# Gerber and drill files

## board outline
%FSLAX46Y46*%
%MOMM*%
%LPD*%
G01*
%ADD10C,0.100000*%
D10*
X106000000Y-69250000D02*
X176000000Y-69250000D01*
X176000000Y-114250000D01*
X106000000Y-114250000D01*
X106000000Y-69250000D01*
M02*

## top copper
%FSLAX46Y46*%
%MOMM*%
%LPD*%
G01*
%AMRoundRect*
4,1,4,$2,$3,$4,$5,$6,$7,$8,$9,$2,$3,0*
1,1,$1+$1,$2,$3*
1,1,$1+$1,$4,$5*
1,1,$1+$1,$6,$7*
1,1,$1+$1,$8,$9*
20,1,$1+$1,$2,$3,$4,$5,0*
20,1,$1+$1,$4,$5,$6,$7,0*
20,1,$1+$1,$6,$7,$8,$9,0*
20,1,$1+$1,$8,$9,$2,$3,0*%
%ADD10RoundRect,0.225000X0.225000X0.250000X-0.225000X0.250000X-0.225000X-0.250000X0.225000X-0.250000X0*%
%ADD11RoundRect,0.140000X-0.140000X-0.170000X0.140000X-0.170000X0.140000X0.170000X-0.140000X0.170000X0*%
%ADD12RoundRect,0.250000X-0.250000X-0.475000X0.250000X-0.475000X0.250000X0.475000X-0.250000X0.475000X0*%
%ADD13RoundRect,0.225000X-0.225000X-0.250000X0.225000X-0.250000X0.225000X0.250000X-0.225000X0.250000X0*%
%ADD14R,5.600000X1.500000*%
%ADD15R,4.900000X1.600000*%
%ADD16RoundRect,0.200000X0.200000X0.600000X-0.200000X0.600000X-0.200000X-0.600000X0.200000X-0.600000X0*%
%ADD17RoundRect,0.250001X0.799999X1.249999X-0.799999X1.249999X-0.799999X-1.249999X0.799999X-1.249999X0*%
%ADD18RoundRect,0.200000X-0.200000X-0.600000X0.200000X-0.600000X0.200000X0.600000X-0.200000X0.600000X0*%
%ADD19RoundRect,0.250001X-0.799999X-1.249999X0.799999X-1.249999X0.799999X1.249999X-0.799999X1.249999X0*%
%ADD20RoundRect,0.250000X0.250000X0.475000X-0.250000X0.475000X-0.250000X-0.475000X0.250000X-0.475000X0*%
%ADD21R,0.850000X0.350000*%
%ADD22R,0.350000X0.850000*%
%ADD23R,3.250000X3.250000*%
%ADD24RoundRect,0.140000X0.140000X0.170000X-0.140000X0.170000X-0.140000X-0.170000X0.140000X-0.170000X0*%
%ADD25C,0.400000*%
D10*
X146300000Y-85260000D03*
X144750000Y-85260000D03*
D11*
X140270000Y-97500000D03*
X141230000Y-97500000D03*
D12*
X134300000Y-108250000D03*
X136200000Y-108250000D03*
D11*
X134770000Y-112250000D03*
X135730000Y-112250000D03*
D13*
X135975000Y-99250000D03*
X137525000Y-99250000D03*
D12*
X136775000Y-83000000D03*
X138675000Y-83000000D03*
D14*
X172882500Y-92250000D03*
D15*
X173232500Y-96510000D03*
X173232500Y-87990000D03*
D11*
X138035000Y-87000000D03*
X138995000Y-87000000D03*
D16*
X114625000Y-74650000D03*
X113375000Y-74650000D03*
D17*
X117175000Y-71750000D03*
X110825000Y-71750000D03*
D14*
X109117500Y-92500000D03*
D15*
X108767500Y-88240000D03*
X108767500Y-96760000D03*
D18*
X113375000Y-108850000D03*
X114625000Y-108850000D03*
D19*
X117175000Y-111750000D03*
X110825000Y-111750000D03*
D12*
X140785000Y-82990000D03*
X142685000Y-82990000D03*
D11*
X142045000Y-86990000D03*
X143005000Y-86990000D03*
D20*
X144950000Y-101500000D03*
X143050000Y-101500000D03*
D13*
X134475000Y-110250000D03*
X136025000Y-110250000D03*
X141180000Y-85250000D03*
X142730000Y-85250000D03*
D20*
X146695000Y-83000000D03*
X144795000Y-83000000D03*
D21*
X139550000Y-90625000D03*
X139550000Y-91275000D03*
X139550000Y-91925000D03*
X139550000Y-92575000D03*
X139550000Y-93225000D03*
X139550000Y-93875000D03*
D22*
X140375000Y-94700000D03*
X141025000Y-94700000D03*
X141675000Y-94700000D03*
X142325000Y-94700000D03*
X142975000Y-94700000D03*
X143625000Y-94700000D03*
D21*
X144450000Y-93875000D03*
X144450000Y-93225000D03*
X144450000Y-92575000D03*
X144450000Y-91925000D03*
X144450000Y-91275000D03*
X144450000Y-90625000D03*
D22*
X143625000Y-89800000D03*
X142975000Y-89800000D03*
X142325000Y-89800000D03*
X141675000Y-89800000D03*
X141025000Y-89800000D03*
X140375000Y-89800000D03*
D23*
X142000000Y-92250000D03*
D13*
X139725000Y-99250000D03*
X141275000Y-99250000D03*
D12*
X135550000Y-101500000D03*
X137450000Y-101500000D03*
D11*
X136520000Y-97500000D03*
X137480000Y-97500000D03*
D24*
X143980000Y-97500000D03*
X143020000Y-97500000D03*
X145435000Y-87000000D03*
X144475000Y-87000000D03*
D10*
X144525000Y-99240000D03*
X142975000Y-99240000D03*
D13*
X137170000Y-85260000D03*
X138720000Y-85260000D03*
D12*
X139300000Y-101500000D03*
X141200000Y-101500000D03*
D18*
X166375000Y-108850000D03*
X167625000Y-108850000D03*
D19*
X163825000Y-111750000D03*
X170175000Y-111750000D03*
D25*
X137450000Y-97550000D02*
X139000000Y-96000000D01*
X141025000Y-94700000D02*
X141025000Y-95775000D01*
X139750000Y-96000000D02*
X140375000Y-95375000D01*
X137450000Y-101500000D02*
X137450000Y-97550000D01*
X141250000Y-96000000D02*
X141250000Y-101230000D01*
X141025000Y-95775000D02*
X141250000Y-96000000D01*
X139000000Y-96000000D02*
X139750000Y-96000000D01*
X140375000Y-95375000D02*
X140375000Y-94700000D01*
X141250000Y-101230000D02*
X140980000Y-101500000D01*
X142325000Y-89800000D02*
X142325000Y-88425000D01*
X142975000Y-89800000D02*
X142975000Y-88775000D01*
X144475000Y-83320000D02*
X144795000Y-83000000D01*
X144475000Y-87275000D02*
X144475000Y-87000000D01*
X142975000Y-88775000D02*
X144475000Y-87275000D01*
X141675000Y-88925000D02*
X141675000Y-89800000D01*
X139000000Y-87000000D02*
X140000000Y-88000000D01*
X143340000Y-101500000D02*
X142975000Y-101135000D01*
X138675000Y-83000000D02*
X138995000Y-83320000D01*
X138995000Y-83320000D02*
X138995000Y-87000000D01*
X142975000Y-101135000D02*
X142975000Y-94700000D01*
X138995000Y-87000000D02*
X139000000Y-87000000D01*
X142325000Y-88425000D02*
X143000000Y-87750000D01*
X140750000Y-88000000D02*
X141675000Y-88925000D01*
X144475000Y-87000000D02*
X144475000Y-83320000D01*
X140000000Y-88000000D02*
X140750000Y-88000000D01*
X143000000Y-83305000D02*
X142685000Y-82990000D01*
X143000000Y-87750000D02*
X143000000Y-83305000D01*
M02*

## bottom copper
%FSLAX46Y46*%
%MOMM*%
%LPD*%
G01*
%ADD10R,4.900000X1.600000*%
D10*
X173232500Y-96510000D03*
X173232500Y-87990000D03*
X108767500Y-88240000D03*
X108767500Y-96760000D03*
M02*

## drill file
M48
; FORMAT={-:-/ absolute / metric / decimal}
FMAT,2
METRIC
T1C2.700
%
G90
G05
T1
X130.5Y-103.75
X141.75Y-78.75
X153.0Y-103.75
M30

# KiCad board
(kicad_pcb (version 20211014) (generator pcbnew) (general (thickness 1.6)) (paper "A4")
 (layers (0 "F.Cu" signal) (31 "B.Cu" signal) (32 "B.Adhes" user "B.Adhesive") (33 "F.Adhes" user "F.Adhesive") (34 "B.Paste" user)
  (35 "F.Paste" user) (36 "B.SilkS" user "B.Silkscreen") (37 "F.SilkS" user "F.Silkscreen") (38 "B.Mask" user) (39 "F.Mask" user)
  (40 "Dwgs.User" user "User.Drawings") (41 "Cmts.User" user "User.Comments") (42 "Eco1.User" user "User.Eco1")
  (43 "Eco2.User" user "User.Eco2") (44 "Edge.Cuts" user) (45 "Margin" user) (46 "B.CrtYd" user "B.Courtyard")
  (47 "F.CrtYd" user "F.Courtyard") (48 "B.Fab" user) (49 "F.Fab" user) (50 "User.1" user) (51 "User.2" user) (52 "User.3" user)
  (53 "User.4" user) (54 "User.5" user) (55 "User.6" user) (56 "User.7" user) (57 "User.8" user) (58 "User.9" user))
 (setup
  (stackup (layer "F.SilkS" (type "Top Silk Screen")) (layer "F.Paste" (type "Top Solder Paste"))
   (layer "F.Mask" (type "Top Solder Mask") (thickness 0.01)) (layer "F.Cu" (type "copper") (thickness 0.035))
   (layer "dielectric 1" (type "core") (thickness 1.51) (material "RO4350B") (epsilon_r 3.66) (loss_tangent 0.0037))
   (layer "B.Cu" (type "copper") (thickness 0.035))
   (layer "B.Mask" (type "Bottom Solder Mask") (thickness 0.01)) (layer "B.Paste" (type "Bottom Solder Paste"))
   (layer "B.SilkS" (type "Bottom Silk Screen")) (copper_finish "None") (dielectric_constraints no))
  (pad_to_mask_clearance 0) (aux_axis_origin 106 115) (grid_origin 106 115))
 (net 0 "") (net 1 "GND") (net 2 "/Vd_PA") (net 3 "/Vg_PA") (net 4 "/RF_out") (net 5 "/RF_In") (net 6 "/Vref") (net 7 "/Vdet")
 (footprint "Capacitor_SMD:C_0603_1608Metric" (layer "F.Cu") (at 145.525 85.26 180)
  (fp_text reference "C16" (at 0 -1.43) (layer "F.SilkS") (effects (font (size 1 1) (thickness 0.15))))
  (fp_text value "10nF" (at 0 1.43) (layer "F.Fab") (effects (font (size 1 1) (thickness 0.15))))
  (pad "1" smd roundrect (at -0.775 0 180) (size 0.9 0.95) (layers "F.Cu" "F.Paste" "F.Mask") (roundrect_rratio 0.25) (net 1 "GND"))
  (pad "2" smd roundrect (at 0.775 0 180) (size 0.9 0.95) (layers "F.Cu" "F.Paste" "F.Mask") (roundrect_rratio 0.25) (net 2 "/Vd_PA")))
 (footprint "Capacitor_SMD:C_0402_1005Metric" (layer "F.Cu") (at 140.75 97.5)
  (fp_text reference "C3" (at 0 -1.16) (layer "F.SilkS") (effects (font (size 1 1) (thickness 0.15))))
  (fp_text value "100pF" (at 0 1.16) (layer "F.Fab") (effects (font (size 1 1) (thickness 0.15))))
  (pad "1" smd roundrect (at -0.48 0) (size 0.56 0.62) (layers "F.Cu" "F.Paste" "F.Mask") (roundrect_rratio 0.25) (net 1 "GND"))
  (pad "2" smd roundrect (at 0.48 0) (size 0.56 0.62) (layers "F.Cu" "F.Paste" "F.Mask") (roundrect_rratio 0.25) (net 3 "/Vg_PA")))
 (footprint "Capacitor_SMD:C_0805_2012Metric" (layer "F.Cu") (at 135.25 108.25)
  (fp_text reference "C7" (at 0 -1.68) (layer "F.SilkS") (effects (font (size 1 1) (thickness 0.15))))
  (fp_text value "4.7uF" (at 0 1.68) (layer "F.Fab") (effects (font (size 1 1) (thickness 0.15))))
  (pad "1" smd roundrect (at -0.95 0) (size 1 1.45) (layers "F.Cu" "F.Paste" "F.Mask") (roundrect_rratio 0.25) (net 1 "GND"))
  (pad "2" smd roundrect (at 0.95 0) (size 1 1.45) (layers "F.Cu" "F.Paste" "F.Mask") (roundrect_rratio 0.25) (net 3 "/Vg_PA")))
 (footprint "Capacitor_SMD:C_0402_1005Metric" (layer "F.Cu") (at 135.25 112.25)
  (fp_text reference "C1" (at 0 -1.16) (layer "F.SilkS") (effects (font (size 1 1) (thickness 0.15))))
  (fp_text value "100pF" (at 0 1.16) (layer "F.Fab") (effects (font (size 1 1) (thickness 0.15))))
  (pad "1" smd roundrect (at -0.48 0) (size 0.56 0.62) (layers "F.Cu" "F.Paste" "F.Mask") (roundrect_rratio 0.25) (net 1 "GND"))
  (pad "2" smd roundrect (at 0.48 0) (size 0.56 0.62) (layers "F.Cu" "F.Paste" "F.Mask") (roundrect_rratio 0.25) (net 3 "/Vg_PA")))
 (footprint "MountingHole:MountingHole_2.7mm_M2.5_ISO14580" (layer "F.Cu") (at 141.75 78.75)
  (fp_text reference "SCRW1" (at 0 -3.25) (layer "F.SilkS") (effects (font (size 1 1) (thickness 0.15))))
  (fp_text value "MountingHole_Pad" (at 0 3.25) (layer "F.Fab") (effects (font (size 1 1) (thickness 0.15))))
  (pad "" np_thru_hole circle (at 0 0) (size 2.7 2.7) (drill 2.7) (layers *.Cu *.Mask)))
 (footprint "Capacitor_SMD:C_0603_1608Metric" (layer "F.Cu") (at 136.75 99.25)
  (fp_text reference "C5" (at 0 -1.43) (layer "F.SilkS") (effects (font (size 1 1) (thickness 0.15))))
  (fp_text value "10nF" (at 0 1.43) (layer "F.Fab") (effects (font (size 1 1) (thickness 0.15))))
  (pad "1" smd roundrect (at -0.775 0) (size 0.9 0.95) (layers "F.Cu" "F.Paste" "F.Mask") (roundrect_rratio 0.25) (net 1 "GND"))
  (pad "2" smd roundrect (at 0.775 0) (size 0.9 0.95) (layers "F.Cu" "F.Paste" "F.Mask") (roundrect_rratio 0.25) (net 3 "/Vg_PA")))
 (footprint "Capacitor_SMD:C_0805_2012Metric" (layer "F.Cu") (at 137.725 83)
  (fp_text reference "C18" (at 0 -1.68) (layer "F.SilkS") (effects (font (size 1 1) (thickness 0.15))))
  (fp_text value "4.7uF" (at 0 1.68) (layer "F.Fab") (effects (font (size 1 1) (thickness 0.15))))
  (pad "1" smd roundrect (at -0.95 0) (size 1 1.45) (layers "F.Cu" "F.Paste" "F.Mask") (roundrect_rratio 0.25) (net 1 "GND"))
  (pad "2" smd roundrect (at 0.95 0) (size 1 1.45) (layers "F.Cu" "F.Paste" "F.Mask") (roundrect_rratio 0.25) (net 2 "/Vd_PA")))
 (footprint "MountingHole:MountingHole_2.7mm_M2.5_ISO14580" (layer "F.Cu") (at 130.5 103.75)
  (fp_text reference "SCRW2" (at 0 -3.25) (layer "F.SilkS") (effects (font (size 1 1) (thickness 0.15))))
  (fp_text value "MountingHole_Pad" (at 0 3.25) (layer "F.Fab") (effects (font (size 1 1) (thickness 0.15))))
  (pad "" np_thru_hole circle (at 0 0) (size 2.7 2.7) (drill 2.7) (layers *.Cu *.Mask)))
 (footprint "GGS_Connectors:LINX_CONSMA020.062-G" (layer "F.Cu") (at 175.6825 92.25 90)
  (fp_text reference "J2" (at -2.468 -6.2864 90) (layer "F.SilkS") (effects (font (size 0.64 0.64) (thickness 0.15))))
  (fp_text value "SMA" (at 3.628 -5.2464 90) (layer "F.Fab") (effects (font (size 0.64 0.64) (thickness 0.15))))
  (pad "1" smd rect (at 0 -2.8 90) (size 1.5 5.6) (layers "F.Cu" "F.Paste" "F.Mask") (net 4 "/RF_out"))
  (pad "S1" smd rect (at -4.26 -2.45 90) (size 1.6 4.9) (layers "F.Cu" "F.Paste" "F.Mask") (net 1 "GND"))
  (pad "S2" smd rect (at 4.26 -2.45 90) (size 1.6 4.9) (layers "F.Cu" "F.Paste" "F.Mask") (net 1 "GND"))
  (pad "S3" smd rect (at -4.26 -2.45 90) (size 1.6 4.9) (layers "B.Cu" "B.Paste" "B.Mask") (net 1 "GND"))
  (pad "S4" smd rect (at 4.26 -2.45 90) (size 1.6 4.9) (layers "B.Cu" "B.Paste" "B.Mask") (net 1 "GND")))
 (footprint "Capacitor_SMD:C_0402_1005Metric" (layer "F.Cu") (at 138.515 87)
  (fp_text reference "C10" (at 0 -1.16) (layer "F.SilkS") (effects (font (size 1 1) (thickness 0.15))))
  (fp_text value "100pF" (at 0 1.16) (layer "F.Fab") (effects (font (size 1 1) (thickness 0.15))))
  (pad "1" smd roundrect (at -0.48 0) (size 0.56 0.62) (layers "F.Cu" "F.Paste" "F.Mask") (roundrect_rratio 0.25) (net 1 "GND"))
  (pad "2" smd roundrect (at 0.48 0) (size 0.56 0.62) (layers "F.Cu" "F.Paste" "F.Mask") (roundrect_rratio 0.25) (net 2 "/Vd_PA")))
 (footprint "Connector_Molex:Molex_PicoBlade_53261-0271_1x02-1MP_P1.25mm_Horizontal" (layer "F.Cu") (at 114 72.25 180)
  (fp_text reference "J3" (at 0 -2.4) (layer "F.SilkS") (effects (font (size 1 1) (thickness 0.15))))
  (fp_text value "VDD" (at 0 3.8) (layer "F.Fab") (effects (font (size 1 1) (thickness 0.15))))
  (pad "1" smd roundrect (at -0.625 -2.4 180) (size 0.8 1.6) (layers "F.Cu" "F.Paste" "F.Mask") (roundrect_rratio 0.25) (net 2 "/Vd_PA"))
  (pad "2" smd roundrect (at 0.625 -2.4 180) (size 0.8 1.6) (layers "F.Cu" "F.Paste" "F.Mask") (roundrect_rratio 0.25) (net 1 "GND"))
  (pad "MP" smd roundrect (at -3.175 0.5 180) (size 2.1 3) (layers "F.Cu" "F.Paste" "F.Mask") (roundrect_rratio 0.119048) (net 1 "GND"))
  (pad "MP" smd roundrect (at 3.175 0.5 180) (size 2.1 3) (layers "F.Cu" "F.Paste" "F.Mask") (roundrect_rratio 0.119048) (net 1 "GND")))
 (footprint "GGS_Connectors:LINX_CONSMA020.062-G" (layer "F.Cu") (at 106.3175 92.5 -90)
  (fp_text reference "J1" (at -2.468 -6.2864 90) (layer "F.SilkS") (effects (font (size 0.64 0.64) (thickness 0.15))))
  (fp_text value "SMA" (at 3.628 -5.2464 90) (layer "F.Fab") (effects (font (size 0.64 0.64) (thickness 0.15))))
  (pad "1" smd rect (at 0 -2.8 270) (size 1.5 5.6) (layers "F.Cu" "F.Paste" "F.Mask") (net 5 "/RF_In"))
  (pad "S1" smd rect (at -4.26 -2.45 270) (size 1.6 4.9) (layers "F.Cu" "F.Paste" "F.Mask") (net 1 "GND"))
  (pad "S2" smd rect (at 4.26 -2.45 270) (size 1.6 4.9) (layers "F.Cu" "F.Paste" "F.Mask") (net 1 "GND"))
  (pad "S3" smd rect (at -4.26 -2.45 270) (size 1.6 4.9) (layers "B.Cu" "B.Paste" "B.Mask") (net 1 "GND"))
  (pad "S4" smd rect (at 4.26 -2.45 270) (size 1.6 4.9) (layers "B.Cu" "B.Paste" "B.Mask") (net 1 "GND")))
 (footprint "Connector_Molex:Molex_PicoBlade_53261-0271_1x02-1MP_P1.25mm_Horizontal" (layer "F.Cu") (at 114 111.25)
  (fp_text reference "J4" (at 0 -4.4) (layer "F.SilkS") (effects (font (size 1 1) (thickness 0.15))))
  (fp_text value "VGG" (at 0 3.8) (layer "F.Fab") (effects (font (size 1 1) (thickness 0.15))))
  (pad "1" smd roundrect (at -0.625 -2.4) (size 0.8 1.6) (layers "F.Cu" "F.Paste" "F.Mask") (roundrect_rratio 0.25) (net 3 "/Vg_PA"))
  (pad "2" smd roundrect (at 0.625 -2.4) (size 0.8 1.6) (layers "F.Cu" "F.Paste" "F.Mask") (roundrect_rratio 0.25) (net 1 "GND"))
  (pad "MP" smd roundrect (at 3.175 0.5) (size 2.1 3) (layers "F.Cu" "F.Paste" "F.Mask") (roundrect_rratio 0.119048) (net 1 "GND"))
  (pad "MP" smd roundrect (at -3.175 0.5) (size 2.1 3) (layers "F.Cu" "F.Paste" "F.Mask") (roundrect_rratio 0.119048) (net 1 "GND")))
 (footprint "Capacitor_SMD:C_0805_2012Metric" (layer "F.Cu") (at 141.735 82.99)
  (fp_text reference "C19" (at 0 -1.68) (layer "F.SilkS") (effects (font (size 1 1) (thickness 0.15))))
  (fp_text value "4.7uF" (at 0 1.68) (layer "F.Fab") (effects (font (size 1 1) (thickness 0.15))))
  (pad "1" smd roundrect (at -0.95 0) (size 1 1.45) (layers "F.Cu" "F.Paste" "F.Mask") (roundrect_rratio 0.25) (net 1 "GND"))
  (pad "2" smd roundrect (at 0.95 0) (size 1 1.45) (layers "F.Cu" "F.Paste" "F.Mask") (roundrect_rratio 0.25) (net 2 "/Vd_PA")))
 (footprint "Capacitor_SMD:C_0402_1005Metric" (layer "F.Cu") (at 142.525 86.99)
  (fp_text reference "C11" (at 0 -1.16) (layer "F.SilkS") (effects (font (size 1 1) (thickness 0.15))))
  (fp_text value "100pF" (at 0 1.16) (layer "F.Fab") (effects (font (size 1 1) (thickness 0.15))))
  (pad "1" smd roundrect (at -0.48 0) (size 0.56 0.62) (layers "F.Cu" "F.Paste" "F.Mask") (roundrect_rratio 0.25) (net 1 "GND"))
  (pad "2" smd roundrect (at 0.48 0) (size 0.56 0.62) (layers "F.Cu" "F.Paste" "F.Mask") (roundrect_rratio 0.25) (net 2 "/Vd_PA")))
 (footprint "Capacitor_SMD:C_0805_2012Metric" (layer "F.Cu") (at 144 101.5 180)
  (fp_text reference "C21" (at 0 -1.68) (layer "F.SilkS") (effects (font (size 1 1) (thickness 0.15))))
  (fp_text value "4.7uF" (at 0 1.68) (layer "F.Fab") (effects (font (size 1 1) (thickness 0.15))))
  (pad "1" smd roundrect (at -0.95 0 180) (size 1 1.45) (layers "F.Cu" "F.Paste" "F.Mask") (roundrect_rratio 0.25) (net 1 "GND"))
  (pad "2" smd roundrect (at 0.95 0 180) (size 1 1.45) (layers "F.Cu" "F.Paste" "F.Mask") (roundrect_rratio 0.25) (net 2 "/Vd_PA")))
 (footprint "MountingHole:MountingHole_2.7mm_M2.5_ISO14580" (layer "F.Cu") (at 153 103.75)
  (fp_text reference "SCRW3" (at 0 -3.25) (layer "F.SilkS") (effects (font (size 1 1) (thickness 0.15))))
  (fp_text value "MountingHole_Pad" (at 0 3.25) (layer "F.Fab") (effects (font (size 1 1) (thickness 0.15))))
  (pad "" np_thru_hole circle (at 0 0) (size 2.7 2.7) (drill 2.7) (layers *.Cu *.Mask)))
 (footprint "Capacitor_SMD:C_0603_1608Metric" (layer "F.Cu") (at 135.25 110.25)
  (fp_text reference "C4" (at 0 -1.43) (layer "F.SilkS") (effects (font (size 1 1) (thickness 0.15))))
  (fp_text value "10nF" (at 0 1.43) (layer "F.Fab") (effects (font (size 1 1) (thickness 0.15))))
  (pad "1" smd roundrect (at -0.775 0) (size 0.9 0.95) (layers "F.Cu" "F.Paste" "F.Mask") (roundrect_rratio 0.25) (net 1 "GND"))
  (pad "2" smd roundrect (at 0.775 0) (size 0.9 0.95) (layers "F.Cu" "F.Paste" "F.Mask") (roundrect_rratio 0.25) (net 3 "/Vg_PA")))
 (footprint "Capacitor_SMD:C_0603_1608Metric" (layer "F.Cu") (at 141.955 85.25)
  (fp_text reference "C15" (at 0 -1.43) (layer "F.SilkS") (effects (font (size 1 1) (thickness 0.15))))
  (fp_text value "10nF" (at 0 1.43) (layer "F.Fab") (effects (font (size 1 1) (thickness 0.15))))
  (pad "1" smd roundrect (at -0.775 0) (size 0.9 0.95) (layers "F.Cu" "F.Paste" "F.Mask") (roundrect_rratio 0.25) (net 1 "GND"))
  (pad "2" smd roundrect (at 0.775 0) (size 0.9 0.95) (layers "F.Cu" "F.Paste" "F.Mask") (roundrect_rratio 0.25) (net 2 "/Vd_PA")))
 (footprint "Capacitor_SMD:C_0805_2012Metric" (layer "F.Cu") (at 145.745 83 180)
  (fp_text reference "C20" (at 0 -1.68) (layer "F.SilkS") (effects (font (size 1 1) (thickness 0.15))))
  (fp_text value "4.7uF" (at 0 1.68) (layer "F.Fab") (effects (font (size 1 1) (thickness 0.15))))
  (pad "1" smd roundrect (at -0.95 0 180) (size 1 1.45) (layers "F.Cu" "F.Paste" "F.Mask") (roundrect_rratio 0.25) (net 1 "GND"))
  (pad "2" smd roundrect (at 0.95 0 180) (size 1 1.45) (layers "F.Cu" "F.Paste" "F.Mask") (roundrect_rratio 0.25) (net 2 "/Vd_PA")))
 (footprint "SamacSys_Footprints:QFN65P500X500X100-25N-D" (layer "F.Cu") (at 142 92.25)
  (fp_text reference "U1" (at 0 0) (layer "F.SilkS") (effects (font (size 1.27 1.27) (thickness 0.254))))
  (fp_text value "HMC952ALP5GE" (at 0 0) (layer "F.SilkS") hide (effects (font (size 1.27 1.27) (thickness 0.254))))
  (pad "1" smd rect locked (at -2.45 -1.625 90) (size 0.35 0.85) (layers "F.Cu" "F.Paste" "F.Mask") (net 1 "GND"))
  (pad "2" smd rect locked (at -2.45 -0.975 90) (size 0.35 0.85) (layers "F.Cu" "F.Paste" "F.Mask") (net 1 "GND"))
  (pad "3" smd rect locked (at -2.45 -0.325 90) (size 0.35 0.85) (layers "F.Cu" "F.Paste" "F.Mask") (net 1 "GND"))
  (pad "4" smd rect locked (at -2.45 0.325 90) (size 0.35 0.85) (layers "F.Cu" "F.Paste" "F.Mask") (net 5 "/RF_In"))
  (pad "5" smd rect locked (at -2.45 0.975 90) (size 0.35 0.85) (layers "F.Cu" "F.Paste" "F.Mask") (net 1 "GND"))
  (pad "6" smd rect locked (at -2.45 1.625 90) (size 0.35 0.85) (layers "F.Cu" "F.Paste" "F.Mask") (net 3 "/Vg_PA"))
  (pad "7" smd rect locked (at -1.625 2.45) (size 0.35 0.85) (layers "F.Cu" "F.Paste" "F.Mask") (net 3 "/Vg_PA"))
  (pad "8" smd rect locked (at -0.975 2.45) (size 0.35 0.85) (layers "F.Cu" "F.Paste" "F.Mask") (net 3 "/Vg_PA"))
  (pad "9" smd rect locked (at -0.325 2.45) (size 0.35 0.85) (layers "F.Cu" "F.Paste" "F.Mask") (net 1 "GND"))
  (pad "10" smd rect locked (at 0.325 2.45) (size 0.35 0.85) (layers "F.Cu" "F.Paste" "F.Mask") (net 1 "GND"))
  (pad "11" smd rect locked (at 0.975 2.45) (size 0.35 0.85) (layers "F.Cu" "F.Paste" "F.Mask") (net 2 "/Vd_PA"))
  (pad "12" smd rect locked (at 1.625 2.45) (size 0.35 0.85) (layers "F.Cu" "F.Paste" "F.Mask") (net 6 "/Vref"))
  (pad "13" smd rect locked (at 2.45 1.625 90) (size 0.35 0.85) (layers "F.Cu" "F.Paste" "F.Mask") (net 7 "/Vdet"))
  (pad "14" smd rect locked (at 2.45 0.975 90) (size 0.35 0.85) (layers "F.Cu" "F.Paste" "F.Mask") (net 1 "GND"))
  (pad "15" smd rect locked (at 2.45 0.325 90) (size 0.35 0.85) (layers "F.Cu" "F.Paste" "F.Mask") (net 1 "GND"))
  (pad "16" smd rect locked (at 2.45 -0.325 90) (size 0.35 0.85) (layers "F.Cu" "F.Paste" "F.Mask") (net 4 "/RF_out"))
  (pad "17" smd rect locked (at 2.45 -0.975 90) (size 0.35 0.85) (layers "F.Cu" "F.Paste" "F.Mask") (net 1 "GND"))
  (pad "18" smd rect locked (at 2.45 -1.625 90) (size 0.35 0.85) (layers "F.Cu" "F.Paste" "F.Mask") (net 1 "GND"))
  (pad "19" smd rect locked (at 1.625 -2.45) (size 0.35 0.85) (layers "F.Cu" "F.Paste" "F.Mask") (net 1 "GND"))
  (pad "20" smd rect locked (at 0.975 -2.45) (size 0.35 0.85) (layers "F.Cu" "F.Paste" "F.Mask") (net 2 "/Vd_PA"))
  (pad "21" smd rect locked (at 0.325 -2.45) (size 0.35 0.85) (layers "F.Cu" "F.Paste" "F.Mask") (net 2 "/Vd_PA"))
  (pad "22" smd rect locked (at -0.325 -2.45) (size 0.35 0.85) (layers "F.Cu" "F.Paste" "F.Mask") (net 2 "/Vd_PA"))
  (pad "23" smd rect locked (at -0.975 -2.45) (size 0.35 0.85) (layers "F.Cu" "F.Paste" "F.Mask") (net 1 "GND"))
  (pad "24" smd rect locked (at -1.625 -2.45) (size 0.35 0.85) (layers "F.Cu" "F.Paste" "F.Mask") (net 1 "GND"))
  (pad "25" smd rect locked (at 0 0) (size 3.25 3.25) (layers "F.Cu" "F.Paste" "F.Mask") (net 1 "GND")))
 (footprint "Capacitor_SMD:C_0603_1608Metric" (layer "F.Cu") (at 140.5 99.25)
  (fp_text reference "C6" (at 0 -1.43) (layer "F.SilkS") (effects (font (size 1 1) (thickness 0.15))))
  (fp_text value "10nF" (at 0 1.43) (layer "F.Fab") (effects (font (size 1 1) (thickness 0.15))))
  (pad "1" smd roundrect (at -0.775 0) (size 0.9 0.95) (layers "F.Cu" "F.Paste" "F.Mask") (roundrect_rratio 0.25) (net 1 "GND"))
  (pad "2" smd roundrect (at 0.775 0) (size 0.9 0.95) (layers "F.Cu" "F.Paste" "F.Mask") (roundrect_rratio 0.25) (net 3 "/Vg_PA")))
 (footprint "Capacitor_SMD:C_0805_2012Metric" (layer "F.Cu") (at 136.5 101.5)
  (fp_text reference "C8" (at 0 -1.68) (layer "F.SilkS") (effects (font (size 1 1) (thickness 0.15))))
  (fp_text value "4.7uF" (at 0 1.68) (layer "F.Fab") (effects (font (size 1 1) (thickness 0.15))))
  (pad "1" smd roundrect (at -0.95 0) (size 1 1.45) (layers "F.Cu" "F.Paste" "F.Mask") (roundrect_rratio 0.25) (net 1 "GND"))
  (pad "2" smd roundrect (at 0.95 0) (size 1 1.45) (layers "F.Cu" "F.Paste" "F.Mask") (roundrect_rratio 0.25) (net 3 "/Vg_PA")))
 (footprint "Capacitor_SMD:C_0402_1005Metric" (layer "F.Cu") (at 137 97.5)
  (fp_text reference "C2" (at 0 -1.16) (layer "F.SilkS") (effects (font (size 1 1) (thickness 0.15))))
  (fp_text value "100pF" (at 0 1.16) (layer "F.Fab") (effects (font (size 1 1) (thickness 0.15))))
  (pad "1" smd roundrect (at -0.48 0) (size 0.56 0.62) (layers "F.Cu" "F.Paste" "F.Mask") (roundrect_rratio 0.25) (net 1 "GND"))
  (pad "2" smd roundrect (at 0.48 0) (size 0.56 0.62) (layers "F.Cu" "F.Paste" "F.Mask") (roundrect_rratio 0.25) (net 3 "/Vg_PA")))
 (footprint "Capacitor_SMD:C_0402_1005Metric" (layer "F.Cu") (at 143.5 97.5 180)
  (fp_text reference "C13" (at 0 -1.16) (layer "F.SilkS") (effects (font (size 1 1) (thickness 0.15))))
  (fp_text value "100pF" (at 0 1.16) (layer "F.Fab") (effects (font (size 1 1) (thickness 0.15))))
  (pad "1" smd roundrect (at -0.48 0 180) (size 0.56 0.62) (layers "F.Cu" "F.Paste" "F.Mask") (roundrect_rratio 0.25) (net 1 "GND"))
  (pad "2" smd roundrect (at 0.48 0 180) (size 0.56 0.62) (layers "F.Cu" "F.Paste" "F.Mask") (roundrect_rratio 0.25) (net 2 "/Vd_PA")))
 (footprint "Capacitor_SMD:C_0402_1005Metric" (layer "F.Cu") (at 144.955 87 180)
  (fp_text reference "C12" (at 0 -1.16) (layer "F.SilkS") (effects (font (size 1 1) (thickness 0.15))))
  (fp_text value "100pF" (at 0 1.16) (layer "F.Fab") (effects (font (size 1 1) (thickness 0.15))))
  (pad "1" smd roundrect (at -0.48 0 180) (size 0.56 0.62) (layers "F.Cu" "F.Paste" "F.Mask") (roundrect_rratio 0.25) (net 1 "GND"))
  (pad "2" smd roundrect (at 0.48 0 180) (size 0.56 0.62) (layers "F.Cu" "F.Paste" "F.Mask") (roundrect_rratio 0.25) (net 2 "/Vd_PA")))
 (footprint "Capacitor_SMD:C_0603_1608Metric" (layer "F.Cu") (at 143.75 99.24 180)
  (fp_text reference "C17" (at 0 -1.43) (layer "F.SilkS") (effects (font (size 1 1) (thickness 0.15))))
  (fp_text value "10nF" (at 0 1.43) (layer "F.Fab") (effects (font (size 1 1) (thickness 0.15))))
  (pad "1" smd roundrect (at -0.775 0 180) (size 0.9 0.95) (layers "F.Cu" "F.Paste" "F.Mask") (roundrect_rratio 0.25) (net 1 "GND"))
  (pad "2" smd roundrect (at 0.775 0 180) (size 0.9 0.95) (layers "F.Cu" "F.Paste" "F.Mask") (roundrect_rratio 0.25) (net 2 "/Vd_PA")))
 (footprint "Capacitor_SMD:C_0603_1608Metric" (layer "F.Cu") (at 137.945 85.26)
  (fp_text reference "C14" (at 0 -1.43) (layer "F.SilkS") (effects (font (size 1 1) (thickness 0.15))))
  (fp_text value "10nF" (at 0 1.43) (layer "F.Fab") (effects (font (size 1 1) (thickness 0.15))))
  (pad "1" smd roundrect (at -0.775 0) (size 0.9 0.95) (layers "F.Cu" "F.Paste" "F.Mask") (roundrect_rratio 0.25) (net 1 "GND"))
  (pad "2" smd roundrect (at 0.775 0) (size 0.9 0.95) (layers "F.Cu" "F.Paste" "F.Mask") (roundrect_rratio 0.25) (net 2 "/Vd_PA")))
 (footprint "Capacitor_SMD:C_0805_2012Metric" (layer "F.Cu") (at 140.25 101.5)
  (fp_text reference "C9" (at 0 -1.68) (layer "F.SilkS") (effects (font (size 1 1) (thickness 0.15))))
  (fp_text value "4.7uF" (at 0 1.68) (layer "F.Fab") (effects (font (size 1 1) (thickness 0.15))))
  (pad "1" smd roundrect (at -0.95 0) (size 1 1.45) (layers "F.Cu" "F.Paste" "F.Mask") (roundrect_rratio 0.25) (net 1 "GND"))
  (pad "2" smd roundrect (at 0.95 0) (size 1 1.45) (layers "F.Cu" "F.Paste" "F.Mask") (roundrect_rratio 0.25) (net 3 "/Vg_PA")))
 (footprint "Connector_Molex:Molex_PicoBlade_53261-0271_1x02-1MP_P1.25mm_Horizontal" (layer "F.Cu") (at 167 111.25)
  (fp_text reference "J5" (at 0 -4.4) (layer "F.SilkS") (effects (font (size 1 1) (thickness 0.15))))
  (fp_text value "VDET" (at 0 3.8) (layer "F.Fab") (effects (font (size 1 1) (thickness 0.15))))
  (pad "1" smd roundrect (at -0.625 -2.4) (size 0.8 1.6) (layers "F.Cu" "F.Paste" "F.Mask") (roundrect_rratio 0.25) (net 7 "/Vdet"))
  (pad "2" smd roundrect (at 0.625 -2.4) (size 0.8 1.6) (layers "F.Cu" "F.Paste" "F.Mask") (roundrect_rratio 0.25) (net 1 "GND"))
  (pad "MP" smd roundrect (at -3.175 0.5) (size 2.1 3) (layers "F.Cu" "F.Paste" "F.Mask") (roundrect_rratio 0.119048) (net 1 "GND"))
  (pad "MP" smd roundrect (at 3.175 0.5) (size 2.1 3) (layers "F.Cu" "F.Paste" "F.Mask") (roundrect_rratio 0.119048) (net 1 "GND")))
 (gr_rect (start 106 114.25) (end 176 69.25) (layer "Edge.Cuts") (width 0.1) (fill none))
 (segment (start 137.45 97.55) (end 139 96) (width 0.4) (layer "F.Cu") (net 3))
 (segment (start 141.025 94.7) (end 141.025 95.775) (width 0.4) (layer "F.Cu") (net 3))
 (segment (start 139.75 96) (end 140.375 95.375) (width 0.4) (layer "F.Cu") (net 3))
 (segment (start 137.45 101.5) (end 137.45 97.55) (width 0.4) (layer "F.Cu") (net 3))
 (segment (start 141.25 96) (end 141.25 101.23) (width 0.4) (layer "F.Cu") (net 3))
 (segment (start 141.025 95.775) (end 141.25 96) (width 0.4) (layer "F.Cu") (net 3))
 (segment (start 139 96) (end 139.75 96) (width 0.4) (layer "F.Cu") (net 3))
 (segment (start 140.375 95.375) (end 140.375 94.7) (width 0.4) (layer "F.Cu") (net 3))
 (segment (start 141.25 101.23) (end 140.98 101.5) (width 0.4) (layer "F.Cu") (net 3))
 (segment (start 142.325 89.8) (end 142.325 88.425) (width 0.4) (layer "F.Cu") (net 2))
 (segment (start 142.975 89.8) (end 142.975 88.775) (width 0.4) (layer "F.Cu") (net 2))
 (segment (start 144.475 83.32) (end 144.795 83) (width 0.4) (layer "F.Cu") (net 2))
 (segment (start 144.475 87.275) (end 144.475 87) (width 0.4) (layer "F.Cu") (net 2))
 (segment (start 142.975 88.775) (end 144.475 87.275) (width 0.4) (layer "F.Cu") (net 2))
 (segment (start 141.675 88.925) (end 141.675 89.8) (width 0.4) (layer "F.Cu") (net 2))
 (segment (start 139 87) (end 140 88) (width 0.4) (layer "F.Cu") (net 2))
 (segment (start 143.34 101.5) (end 142.975 101.135) (width 0.4) (layer "F.Cu") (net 2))
 (segment (start 138.675 83) (end 138.995 83.32) (width 0.4) (layer "F.Cu") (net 2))
 (segment (start 138.995 83.32) (end 138.995 87) (width 0.4) (layer "F.Cu") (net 2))
 (segment (start 142.975 101.135) (end 142.975 94.7) (width 0.4) (layer "F.Cu") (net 2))
 (segment (start 138.995 87) (end 139 87) (width 0.4) (layer "F.Cu") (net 2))
 (segment (start 142.325 88.425) (end 143 87.75) (width 0.4) (layer "F.Cu") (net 2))
 (segment (start 140.75 88) (end 141.675 88.925) (width 0.4) (layer "F.Cu") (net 2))
 (segment (start 144.475 87) (end 144.475 83.32) (width 0.4) (layer "F.Cu") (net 2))
 (segment (start 140 88) (end 140.75 88) (width 0.4) (layer "F.Cu") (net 2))
 (segment (start 143 83.305) (end 142.685 82.99) (width 0.4) (layer "F.Cu") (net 2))
 (segment (start 143 87.75) (end 143 83.305) (width 0.4) (layer "F.Cu") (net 2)))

